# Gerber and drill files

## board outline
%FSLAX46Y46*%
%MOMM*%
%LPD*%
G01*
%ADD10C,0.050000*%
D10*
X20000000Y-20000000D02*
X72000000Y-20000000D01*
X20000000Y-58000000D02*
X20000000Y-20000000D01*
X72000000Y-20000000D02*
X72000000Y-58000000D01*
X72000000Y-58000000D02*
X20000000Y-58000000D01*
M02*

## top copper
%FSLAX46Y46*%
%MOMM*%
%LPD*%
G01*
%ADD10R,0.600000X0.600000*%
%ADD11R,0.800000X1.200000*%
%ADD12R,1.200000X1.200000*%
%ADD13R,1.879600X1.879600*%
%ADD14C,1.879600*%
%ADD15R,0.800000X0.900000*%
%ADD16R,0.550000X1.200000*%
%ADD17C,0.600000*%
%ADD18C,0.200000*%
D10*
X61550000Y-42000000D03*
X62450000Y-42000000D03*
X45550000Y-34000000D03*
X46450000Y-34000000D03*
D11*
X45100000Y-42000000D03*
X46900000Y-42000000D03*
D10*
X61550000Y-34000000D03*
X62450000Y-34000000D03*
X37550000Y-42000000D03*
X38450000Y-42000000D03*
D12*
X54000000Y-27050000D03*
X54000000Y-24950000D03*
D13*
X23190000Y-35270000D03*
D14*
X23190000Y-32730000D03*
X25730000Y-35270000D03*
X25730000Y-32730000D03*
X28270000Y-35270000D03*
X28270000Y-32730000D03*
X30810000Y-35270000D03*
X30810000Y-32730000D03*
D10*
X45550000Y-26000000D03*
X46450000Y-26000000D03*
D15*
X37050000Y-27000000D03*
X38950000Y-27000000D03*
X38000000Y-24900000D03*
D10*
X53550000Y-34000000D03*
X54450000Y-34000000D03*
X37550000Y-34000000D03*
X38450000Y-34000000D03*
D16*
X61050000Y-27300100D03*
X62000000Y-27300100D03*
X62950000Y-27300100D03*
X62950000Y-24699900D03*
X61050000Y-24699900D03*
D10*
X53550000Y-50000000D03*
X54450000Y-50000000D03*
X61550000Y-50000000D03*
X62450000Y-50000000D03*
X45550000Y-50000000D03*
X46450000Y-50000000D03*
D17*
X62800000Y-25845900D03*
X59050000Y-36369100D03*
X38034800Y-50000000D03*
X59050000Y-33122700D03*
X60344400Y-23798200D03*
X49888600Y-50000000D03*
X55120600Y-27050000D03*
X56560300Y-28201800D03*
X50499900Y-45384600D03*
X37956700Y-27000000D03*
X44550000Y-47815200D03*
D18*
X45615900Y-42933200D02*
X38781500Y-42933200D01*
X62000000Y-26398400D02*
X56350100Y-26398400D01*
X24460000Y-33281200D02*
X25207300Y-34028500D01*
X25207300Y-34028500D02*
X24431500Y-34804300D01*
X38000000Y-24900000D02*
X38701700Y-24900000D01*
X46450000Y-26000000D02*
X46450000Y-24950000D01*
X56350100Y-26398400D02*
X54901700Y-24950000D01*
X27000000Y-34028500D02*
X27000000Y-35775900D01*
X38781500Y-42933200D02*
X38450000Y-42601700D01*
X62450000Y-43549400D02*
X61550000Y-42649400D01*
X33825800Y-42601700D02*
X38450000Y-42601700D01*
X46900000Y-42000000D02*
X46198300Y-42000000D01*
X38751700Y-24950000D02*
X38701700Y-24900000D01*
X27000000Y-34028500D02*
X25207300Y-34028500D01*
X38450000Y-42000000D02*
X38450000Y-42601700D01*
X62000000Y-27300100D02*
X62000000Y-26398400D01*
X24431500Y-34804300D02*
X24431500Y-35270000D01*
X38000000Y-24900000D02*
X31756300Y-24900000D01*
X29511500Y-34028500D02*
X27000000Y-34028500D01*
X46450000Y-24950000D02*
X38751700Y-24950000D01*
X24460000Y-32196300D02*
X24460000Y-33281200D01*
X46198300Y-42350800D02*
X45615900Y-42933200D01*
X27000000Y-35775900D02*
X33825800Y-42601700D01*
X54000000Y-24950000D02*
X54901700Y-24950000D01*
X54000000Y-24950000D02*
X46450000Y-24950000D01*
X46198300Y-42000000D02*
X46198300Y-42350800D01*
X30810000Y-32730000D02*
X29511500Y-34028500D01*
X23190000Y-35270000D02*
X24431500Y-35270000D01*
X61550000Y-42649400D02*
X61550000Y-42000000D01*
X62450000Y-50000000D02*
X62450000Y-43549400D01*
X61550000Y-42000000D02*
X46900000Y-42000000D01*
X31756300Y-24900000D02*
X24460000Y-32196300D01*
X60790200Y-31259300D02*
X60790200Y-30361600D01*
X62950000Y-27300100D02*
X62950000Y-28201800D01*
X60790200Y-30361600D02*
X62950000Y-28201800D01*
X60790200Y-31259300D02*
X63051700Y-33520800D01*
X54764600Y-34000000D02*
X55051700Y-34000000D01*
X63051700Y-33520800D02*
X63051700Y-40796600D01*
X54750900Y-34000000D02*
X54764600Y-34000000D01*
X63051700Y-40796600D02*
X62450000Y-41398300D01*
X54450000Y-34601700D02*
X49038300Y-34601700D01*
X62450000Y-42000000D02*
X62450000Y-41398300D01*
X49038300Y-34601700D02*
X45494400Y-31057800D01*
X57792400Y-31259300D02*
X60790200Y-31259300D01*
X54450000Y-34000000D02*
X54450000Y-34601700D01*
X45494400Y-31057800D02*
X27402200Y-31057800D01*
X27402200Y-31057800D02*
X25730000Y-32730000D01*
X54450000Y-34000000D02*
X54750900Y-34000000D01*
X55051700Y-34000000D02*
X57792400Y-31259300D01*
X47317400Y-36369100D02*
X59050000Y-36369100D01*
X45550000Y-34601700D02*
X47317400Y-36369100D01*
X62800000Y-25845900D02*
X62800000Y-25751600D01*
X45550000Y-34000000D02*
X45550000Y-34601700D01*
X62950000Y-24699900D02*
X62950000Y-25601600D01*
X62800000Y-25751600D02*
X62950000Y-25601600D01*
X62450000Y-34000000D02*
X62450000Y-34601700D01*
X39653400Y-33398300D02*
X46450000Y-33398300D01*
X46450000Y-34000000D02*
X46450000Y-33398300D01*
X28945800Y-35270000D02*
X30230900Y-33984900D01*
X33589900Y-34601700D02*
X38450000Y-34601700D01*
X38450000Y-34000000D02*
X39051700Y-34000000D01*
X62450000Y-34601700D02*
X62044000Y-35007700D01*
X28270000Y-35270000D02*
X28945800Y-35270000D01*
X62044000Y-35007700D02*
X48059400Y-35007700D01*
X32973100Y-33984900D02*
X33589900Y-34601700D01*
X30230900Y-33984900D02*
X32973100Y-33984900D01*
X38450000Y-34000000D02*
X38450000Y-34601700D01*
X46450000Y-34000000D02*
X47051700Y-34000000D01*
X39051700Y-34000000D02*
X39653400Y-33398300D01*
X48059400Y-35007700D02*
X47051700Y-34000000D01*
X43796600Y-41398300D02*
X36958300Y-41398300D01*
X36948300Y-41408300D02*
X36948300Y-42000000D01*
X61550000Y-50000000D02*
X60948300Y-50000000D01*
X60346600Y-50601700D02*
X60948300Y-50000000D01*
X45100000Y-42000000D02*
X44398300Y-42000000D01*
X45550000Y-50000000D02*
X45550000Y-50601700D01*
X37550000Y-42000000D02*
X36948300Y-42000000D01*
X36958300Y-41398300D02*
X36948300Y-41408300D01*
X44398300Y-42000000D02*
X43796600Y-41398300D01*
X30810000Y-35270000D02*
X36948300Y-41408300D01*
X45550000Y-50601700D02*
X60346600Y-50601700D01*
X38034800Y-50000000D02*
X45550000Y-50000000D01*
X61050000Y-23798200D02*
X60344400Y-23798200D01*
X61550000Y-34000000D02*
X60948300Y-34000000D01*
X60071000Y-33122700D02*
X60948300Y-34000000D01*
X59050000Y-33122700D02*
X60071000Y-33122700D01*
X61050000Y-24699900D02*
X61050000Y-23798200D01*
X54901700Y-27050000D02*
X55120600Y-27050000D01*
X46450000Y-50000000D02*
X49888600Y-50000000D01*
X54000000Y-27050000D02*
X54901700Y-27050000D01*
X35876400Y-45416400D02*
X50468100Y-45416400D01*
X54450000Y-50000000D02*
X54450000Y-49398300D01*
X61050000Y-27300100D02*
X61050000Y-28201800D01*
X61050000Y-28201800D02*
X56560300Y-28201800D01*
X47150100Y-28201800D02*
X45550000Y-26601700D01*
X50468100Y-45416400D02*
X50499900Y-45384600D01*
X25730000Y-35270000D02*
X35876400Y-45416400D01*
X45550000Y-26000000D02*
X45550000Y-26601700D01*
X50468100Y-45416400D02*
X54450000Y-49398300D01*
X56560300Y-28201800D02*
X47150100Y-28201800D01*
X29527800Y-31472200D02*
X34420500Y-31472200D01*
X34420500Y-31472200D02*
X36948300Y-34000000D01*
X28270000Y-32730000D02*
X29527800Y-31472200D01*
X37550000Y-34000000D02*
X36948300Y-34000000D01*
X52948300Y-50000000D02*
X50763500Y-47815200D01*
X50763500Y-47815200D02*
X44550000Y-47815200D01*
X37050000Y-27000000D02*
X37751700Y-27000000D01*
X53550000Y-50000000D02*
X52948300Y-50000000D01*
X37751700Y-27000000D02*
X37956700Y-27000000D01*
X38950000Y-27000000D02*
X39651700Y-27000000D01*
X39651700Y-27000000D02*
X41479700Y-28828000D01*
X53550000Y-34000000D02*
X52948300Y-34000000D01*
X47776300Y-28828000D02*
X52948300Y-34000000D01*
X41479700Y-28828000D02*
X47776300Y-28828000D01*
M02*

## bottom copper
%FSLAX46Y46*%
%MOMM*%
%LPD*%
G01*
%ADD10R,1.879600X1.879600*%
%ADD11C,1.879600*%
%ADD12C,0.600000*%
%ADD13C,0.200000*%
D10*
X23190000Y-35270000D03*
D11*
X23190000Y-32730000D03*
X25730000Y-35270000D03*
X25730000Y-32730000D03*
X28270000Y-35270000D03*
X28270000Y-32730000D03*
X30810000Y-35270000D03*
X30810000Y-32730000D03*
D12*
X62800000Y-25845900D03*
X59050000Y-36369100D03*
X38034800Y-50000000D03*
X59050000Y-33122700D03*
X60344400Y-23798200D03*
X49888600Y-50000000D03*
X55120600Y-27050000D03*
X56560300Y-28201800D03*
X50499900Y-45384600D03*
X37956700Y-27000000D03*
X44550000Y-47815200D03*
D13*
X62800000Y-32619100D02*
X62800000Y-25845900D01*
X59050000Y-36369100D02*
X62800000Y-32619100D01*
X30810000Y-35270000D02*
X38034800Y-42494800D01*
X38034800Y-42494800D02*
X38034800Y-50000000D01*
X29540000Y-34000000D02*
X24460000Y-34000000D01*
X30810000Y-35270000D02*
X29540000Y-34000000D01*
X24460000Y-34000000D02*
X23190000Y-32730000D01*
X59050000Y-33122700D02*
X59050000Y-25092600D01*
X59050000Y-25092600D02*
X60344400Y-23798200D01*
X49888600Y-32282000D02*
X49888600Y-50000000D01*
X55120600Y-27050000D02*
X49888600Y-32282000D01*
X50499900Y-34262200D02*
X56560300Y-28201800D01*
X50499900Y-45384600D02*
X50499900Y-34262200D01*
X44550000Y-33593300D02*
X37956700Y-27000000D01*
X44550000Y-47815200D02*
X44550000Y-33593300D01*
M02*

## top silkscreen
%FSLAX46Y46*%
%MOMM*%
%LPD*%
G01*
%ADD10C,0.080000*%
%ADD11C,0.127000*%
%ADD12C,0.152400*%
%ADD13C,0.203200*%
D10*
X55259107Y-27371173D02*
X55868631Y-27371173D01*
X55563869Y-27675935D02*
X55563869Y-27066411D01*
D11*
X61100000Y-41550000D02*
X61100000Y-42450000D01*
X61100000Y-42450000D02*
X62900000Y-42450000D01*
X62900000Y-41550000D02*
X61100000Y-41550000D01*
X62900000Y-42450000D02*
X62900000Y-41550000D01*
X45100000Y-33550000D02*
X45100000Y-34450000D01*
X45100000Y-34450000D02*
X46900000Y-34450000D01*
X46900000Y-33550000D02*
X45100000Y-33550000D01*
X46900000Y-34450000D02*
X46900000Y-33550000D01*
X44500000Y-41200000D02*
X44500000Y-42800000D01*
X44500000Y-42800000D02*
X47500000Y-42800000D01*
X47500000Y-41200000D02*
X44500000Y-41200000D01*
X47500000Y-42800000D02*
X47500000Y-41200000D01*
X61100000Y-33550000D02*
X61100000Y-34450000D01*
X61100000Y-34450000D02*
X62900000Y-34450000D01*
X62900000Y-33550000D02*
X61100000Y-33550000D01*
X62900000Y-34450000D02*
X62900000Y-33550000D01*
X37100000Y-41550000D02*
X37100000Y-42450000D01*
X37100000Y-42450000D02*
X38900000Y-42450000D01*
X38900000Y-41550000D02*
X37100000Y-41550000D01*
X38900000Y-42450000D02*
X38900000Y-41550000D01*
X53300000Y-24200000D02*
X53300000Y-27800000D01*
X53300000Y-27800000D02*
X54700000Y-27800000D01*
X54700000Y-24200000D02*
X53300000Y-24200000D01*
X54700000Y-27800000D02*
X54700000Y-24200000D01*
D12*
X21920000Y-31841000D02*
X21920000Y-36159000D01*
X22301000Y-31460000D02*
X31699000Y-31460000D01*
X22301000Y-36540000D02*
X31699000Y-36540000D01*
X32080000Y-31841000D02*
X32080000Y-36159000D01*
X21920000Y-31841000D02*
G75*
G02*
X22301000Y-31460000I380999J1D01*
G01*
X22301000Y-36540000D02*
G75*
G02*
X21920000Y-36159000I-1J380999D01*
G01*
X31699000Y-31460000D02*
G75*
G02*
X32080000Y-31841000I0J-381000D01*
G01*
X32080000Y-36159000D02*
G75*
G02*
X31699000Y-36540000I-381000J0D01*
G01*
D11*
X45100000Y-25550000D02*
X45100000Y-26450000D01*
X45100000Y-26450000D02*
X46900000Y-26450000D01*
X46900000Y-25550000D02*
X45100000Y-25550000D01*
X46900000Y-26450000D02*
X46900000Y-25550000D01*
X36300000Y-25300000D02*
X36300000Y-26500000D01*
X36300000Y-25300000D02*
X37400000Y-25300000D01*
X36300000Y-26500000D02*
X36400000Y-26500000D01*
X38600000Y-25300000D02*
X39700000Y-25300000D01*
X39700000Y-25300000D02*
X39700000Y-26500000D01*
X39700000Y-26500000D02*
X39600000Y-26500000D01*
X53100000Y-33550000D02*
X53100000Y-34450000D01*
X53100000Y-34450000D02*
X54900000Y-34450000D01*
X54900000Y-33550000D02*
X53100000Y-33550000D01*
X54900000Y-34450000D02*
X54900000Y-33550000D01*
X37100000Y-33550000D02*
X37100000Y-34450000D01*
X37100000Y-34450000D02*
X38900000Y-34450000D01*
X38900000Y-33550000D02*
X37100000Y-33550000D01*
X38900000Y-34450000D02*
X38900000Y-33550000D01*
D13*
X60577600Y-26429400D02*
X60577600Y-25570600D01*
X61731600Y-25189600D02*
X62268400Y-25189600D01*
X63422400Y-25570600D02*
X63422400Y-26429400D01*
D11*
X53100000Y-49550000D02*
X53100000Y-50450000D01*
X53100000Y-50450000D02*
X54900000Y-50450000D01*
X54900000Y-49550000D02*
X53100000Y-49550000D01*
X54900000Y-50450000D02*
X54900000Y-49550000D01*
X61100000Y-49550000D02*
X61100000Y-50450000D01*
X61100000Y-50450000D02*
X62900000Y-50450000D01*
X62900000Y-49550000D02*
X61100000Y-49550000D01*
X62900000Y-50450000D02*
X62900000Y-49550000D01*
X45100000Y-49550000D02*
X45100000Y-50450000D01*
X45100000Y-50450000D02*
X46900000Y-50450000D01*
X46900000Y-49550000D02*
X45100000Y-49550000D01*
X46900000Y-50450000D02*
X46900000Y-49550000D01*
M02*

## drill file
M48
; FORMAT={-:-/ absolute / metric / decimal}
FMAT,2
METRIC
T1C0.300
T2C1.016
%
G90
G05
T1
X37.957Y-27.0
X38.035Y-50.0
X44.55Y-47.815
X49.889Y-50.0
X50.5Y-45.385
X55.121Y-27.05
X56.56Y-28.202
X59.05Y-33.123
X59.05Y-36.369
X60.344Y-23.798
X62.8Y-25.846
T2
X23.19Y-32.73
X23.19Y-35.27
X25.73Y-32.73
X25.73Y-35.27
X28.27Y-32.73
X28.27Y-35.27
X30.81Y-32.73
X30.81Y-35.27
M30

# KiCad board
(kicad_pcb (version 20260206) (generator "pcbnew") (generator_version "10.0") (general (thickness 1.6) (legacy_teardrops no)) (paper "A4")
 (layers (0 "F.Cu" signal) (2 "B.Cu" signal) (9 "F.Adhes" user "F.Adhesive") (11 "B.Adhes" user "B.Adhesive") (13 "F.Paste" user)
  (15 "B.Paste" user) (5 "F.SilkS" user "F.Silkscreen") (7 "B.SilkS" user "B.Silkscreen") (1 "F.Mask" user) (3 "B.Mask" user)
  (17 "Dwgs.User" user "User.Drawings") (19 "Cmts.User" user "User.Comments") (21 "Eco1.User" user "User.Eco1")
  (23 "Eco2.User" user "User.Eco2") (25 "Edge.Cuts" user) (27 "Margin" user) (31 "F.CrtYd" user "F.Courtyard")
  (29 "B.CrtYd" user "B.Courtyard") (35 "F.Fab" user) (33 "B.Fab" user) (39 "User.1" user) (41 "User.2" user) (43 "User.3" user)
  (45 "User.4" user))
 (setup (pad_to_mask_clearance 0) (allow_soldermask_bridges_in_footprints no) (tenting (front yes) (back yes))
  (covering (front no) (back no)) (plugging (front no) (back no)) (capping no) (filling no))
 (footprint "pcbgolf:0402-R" (layer "F.Cu") (at 62 42)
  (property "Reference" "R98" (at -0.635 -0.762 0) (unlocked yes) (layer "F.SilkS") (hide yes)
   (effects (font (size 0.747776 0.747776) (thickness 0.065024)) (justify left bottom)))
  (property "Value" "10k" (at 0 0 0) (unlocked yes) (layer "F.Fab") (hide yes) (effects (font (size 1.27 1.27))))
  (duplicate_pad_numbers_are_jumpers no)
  (fp_line (start -0.9 -0.45) (end -0.9 0.45) (stroke (width 0.127) (type solid)) (layer "F.SilkS"))
  (fp_line (start -0.9 0.45) (end 0.9 0.45) (stroke (width 0.127) (type solid)) (layer "F.SilkS"))
  (fp_line (start 0.9 -0.45) (end -0.9 -0.45) (stroke (width 0.127) (type solid)) (layer "F.SilkS"))
  (fp_line (start 0.9 0.45) (end 0.9 -0.45) (stroke (width 0.127) (type solid)) (layer "F.SilkS"))
  (pad "1" smd rect (at -0.45 0) (size 0.6 0.6) (layers "F.Cu" "F.Mask" "F.Paste") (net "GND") (solder_mask_margin 0.0508)
   (solder_paste_margin 0) (thermal_bridge_angle 0))
  (pad "2" smd rect (at 0.45 0) (size 0.6 0.6) (layers "F.Cu" "F.Mask" "F.Paste") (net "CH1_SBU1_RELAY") (solder_mask_margin 0.0508)
   (solder_paste_margin 0) (thermal_bridge_angle 0)))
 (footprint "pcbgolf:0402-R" (layer "F.Cu") (at 46 34)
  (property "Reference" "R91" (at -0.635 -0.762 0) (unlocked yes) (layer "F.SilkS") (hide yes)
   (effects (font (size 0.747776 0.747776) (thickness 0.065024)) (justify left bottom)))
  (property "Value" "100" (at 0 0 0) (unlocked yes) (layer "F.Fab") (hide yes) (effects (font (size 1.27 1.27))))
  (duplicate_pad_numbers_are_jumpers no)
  (fp_line (start -0.9 -0.45) (end -0.9 0.45) (stroke (width 0.127) (type solid)) (layer "F.SilkS"))
  (fp_line (start -0.9 0.45) (end 0.9 0.45) (stroke (width 0.127) (type solid)) (layer "F.SilkS"))
  (fp_line (start 0.9 -0.45) (end -0.9 -0.45) (stroke (width 0.127) (type solid)) (layer "F.SilkS"))
  (fp_line (start 0.9 0.45) (end 0.9 -0.45) (stroke (width 0.127) (type solid)) (layer "F.SilkS"))
  (pad "1" smd rect (at -0.45 0) (size 0.6 0.6) (layers "F.Cu" "F.Mask" "F.Paste") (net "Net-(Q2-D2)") (solder_mask_margin 0.0508)
   (solder_paste_margin 0) (thermal_bridge_angle 0))
  (pad "2" smd rect (at 0.45 0) (size 0.6 0.6) (layers "F.Cu" "F.Mask" "F.Paste") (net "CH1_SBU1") (solder_mask_margin 0.0508)
   (solder_paste_margin 0) (thermal_bridge_angle 0)))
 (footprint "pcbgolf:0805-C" (layer "F.Cu") (at 46 42)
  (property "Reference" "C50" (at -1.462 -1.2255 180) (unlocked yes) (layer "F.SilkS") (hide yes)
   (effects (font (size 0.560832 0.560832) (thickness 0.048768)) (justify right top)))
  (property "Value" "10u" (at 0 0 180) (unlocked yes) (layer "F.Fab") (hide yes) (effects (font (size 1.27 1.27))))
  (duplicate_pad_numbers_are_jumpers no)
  (fp_line (start -1.5 -0.8) (end -1.5 0.8) (stroke (width 0.127) (type solid)) (layer "F.SilkS"))
  (fp_line (start -1.5 0.8) (end 1.5 0.8) (stroke (width 0.127) (type solid)) (layer "F.SilkS"))
  (fp_line (start 1.5 -0.8) (end -1.5 -0.8) (stroke (width 0.127) (type solid)) (layer "F.SilkS"))
  (fp_line (start 1.5 0.8) (end 1.5 -0.8) (stroke (width 0.127) (type solid)) (layer "F.SilkS"))
  (pad "1" smd rect (at -0.9 0) (size 0.8 1.2) (layers "F.Cu" "F.Mask" "F.Paste") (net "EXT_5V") (solder_mask_margin 0.0508)
   (solder_paste_margin 0) (thermal_bridge_angle 0))
  (pad "2" smd rect (at 0.9 0) (size 0.8 1.2) (layers "F.Cu" "F.Mask" "F.Paste") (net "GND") (solder_mask_margin 0.0508)
   (solder_paste_margin 0) (thermal_bridge_angle 0)))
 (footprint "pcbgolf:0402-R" (layer "F.Cu") (at 62 34)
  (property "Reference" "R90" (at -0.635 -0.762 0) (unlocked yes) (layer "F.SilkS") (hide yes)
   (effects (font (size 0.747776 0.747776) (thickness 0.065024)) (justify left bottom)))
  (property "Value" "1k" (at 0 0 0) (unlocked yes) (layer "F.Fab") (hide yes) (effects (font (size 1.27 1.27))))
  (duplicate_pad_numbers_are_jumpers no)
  (fp_line (start -0.9 -0.45) (end -0.9 0.45) (stroke (width 0.127) (type solid)) (layer "F.SilkS"))
  (fp_line (start -0.9 0.45) (end 0.9 0.45) (stroke (width 0.127) (type solid)) (layer "F.SilkS"))
  (fp_line (start 0.9 -0.45) (end -0.9 -0.45) (stroke (width 0.127) (type solid)) (layer "F.SilkS"))
  (fp_line (start 0.9 0.45) (end 0.9 -0.45) (stroke (width 0.127) (type solid)) (layer "F.SilkS"))
  (pad "1" smd rect (at -0.45 0) (size 0.6 0.6) (layers "F.Cu" "F.Mask" "F.Paste") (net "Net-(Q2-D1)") (solder_mask_margin 0.0508)
   (solder_paste_margin 0) (thermal_bridge_angle 0))
  (pad "2" smd rect (at 0.45 0) (size 0.6 0.6) (layers "F.Cu" "F.Mask" "F.Paste") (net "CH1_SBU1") (solder_mask_margin 0.0508)
   (solder_paste_margin 0) (thermal_bridge_angle 0)))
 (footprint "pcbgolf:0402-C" (layer "F.Cu") (at 38 42)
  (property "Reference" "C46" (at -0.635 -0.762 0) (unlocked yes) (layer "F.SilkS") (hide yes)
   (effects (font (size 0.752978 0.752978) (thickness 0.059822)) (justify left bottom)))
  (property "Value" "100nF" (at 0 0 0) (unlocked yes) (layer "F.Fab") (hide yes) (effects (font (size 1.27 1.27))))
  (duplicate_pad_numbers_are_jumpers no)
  (fp_line (start -0.9 -0.45) (end -0.9 0.45) (stroke (width 0.127) (type solid)) (layer "F.SilkS"))
  (fp_line (start -0.9 0.45) (end 0.9 0.45) (stroke (width 0.127) (type solid)) (layer "F.SilkS"))
  (fp_line (start 0.9 -0.45) (end -0.9 -0.45) (stroke (width 0.127) (type solid)) (layer "F.SilkS"))
  (fp_line (start 0.9 0.45) (end 0.9 -0.45) (stroke (width 0.127) (type solid)) (layer "F.SilkS"))
  (pad "1" smd rect (at -0.45 0) (size 0.6 0.6) (layers "F.Cu" "F.Mask" "F.Paste") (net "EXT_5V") (solder_mask_margin 0.0508)
   (solder_paste_margin 0) (thermal_bridge_angle 0))
  (pad "2" smd rect (at 0.45 0) (size 0.6 0.6) (layers "F.Cu" "F.Mask" "F.Paste") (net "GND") (solder_mask_margin 0.0508)
   (solder_paste_margin 0) (thermal_bridge_angle 0)))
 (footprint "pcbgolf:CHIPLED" (layer "F.Cu") (at 54 26)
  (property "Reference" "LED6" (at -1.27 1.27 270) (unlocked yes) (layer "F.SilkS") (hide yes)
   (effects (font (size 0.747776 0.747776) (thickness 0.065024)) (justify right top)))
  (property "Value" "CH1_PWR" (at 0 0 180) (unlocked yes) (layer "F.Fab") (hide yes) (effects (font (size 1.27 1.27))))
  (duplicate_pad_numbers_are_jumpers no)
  (fp_line (start -0.7 -1.8) (end -0.7 1.8) (stroke (width 0.127) (type solid)) (layer "F.SilkS"))
  (fp_line (start -0.7 1.8) (end 0.7 1.8) (stroke (width 0.127) (type solid)) (layer "F.SilkS"))
  (fp_line (start 0.7 -1.8) (end -0.7 -1.8) (stroke (width 0.127) (type solid)) (layer "F.SilkS"))
  (fp_line (start 0.7 1.8) (end 0.7 -1.8) (stroke (width 0.127) (type solid)) (layer "F.SilkS"))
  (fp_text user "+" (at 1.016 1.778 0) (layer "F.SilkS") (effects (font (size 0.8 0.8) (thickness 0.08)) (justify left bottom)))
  (pad "A" smd rect (at 0 1.05) (size 1.2 1.2) (layers "F.Cu" "F.Mask" "F.Paste") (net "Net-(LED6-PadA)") (solder_mask_margin 0.0508)
   (solder_paste_margin 0) (thermal_bridge_angle 0))
  (pad "C" smd rect (at 0 -1.05) (size 1.2 1.2) (layers "F.Cu" "F.Mask" "F.Paste") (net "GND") (solder_mask_margin 0.0508)
   (solder_paste_margin 0) (thermal_bridge_angle 0)))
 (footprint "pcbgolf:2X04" (layer "F.Cu") (at 27 34)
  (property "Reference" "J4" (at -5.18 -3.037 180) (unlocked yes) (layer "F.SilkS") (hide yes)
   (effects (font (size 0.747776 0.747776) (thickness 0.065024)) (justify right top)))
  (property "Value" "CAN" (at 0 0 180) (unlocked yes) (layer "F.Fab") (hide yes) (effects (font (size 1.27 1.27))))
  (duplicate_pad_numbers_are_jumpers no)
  (fp_line (start -5.08 -2.159) (end -5.08 2.159) (stroke (width 0.1524) (type solid)) (layer "F.SilkS"))
  (fp_line (start -4.699 -2.54) (end 4.699 -2.54) (stroke (width 0.1524) (type solid)) (layer "F.SilkS"))
  (fp_line (start -4.699 2.54) (end 4.699 2.54) (stroke (width 0.1524) (type solid)) (layer "F.SilkS"))
  (fp_line (start 5.08 -2.159) (end 5.08 2.159) (stroke (width 0.1524) (type solid)) (layer "F.SilkS"))
  (fp_arc (start -5.08 -2.159) (mid -4.968408 -2.428408) (end -4.699 -2.54) (stroke (width 0.1524) (type solid)) (layer "F.SilkS"))
  (fp_arc (start -4.699 2.54) (mid -4.968408 2.428408) (end -5.08 2.159) (stroke (width 0.1524) (type solid)) (layer "F.SilkS"))
  (fp_arc (start 4.699 -2.54) (mid 4.968408 -2.428408) (end 5.08 -2.159) (stroke (width 0.1524) (type solid)) (layer "F.SilkS"))
  (fp_arc (start 5.08 2.159) (mid 4.968408 2.428408) (end 4.699 2.54) (stroke (width 0.1524) (type solid)) (layer "F.SilkS"))
  (pad "1" thru_hole rect (at -3.81 1.27 90) (size 1.8796 1.8796) (drill 1.016) (layers "*.Cu" "*.Mask") (remove_unused_layers no)
   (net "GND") (solder_mask_margin 0.0508) (thermal_bridge_angle 0))
  (pad "2" thru_hole circle (at -3.81 -1.27 90) (size 1.8796 1.8796) (drill 1.016) (layers "*.Cu" "*.Mask") (remove_unused_layers no)
   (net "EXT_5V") (solder_mask_margin 0.0508) (thermal_bridge_angle 0))
  (pad "3" thru_hole circle (at -1.27 1.27 90) (size 1.8796 1.8796) (drill 1.016) (layers "*.Cu" "*.Mask") (remove_unused_layers no)
   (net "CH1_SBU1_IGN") (solder_mask_margin 0.0508) (thermal_bridge_angle 0))
  (pad "4" thru_hole circle (at -1.27 -1.27 90) (size 1.8796 1.8796) (drill 1.016) (layers "*.Cu" "*.Mask") (remove_unused_layers no)
   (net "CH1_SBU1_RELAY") (solder_mask_margin 0.0508) (thermal_bridge_angle 0))
  (pad "5" thru_hole circle (at 1.27 1.27 90) (size 1.8796 1.8796) (drill 1.016) (layers "*.Cu" "*.Mask") (remove_unused_layers no)
   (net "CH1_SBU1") (solder_mask_margin 0.0508) (thermal_bridge_angle 0))
  (pad "6" thru_hole circle (at 1.27 -1.27 90) (size 1.8796 1.8796) (drill 1.016) (layers "*.Cu" "*.Mask") (remove_unused_layers no)
   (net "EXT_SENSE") (solder_mask_margin 0.0508) (thermal_bridge_angle 0))
  (pad "7" thru_hole circle (at 3.81 1.27 90) (size 1.8796 1.8796) (drill 1.016) (layers "*.Cu" "*.Mask") (remove_unused_layers no)
   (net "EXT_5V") (solder_mask_margin 0.0508) (thermal_bridge_angle 0))
  (pad "8" thru_hole circle (at 3.81 -1.27 90) (size 1.8796 1.8796) (drill 1.016) (layers "*.Cu" "*.Mask") (remove_unused_layers no)
   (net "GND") (solder_mask_margin 0.0508) (thermal_bridge_angle 0)))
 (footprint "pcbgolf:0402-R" (layer "F.Cu") (at 46 26)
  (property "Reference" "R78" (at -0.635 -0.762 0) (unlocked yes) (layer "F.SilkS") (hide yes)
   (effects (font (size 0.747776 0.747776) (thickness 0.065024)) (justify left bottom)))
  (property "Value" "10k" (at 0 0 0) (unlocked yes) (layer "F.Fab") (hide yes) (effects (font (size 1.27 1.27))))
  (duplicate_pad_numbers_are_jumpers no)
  (fp_line (start -0.9 -0.45) (end -0.9 0.45) (stroke (width 0.127) (type solid)) (layer "F.SilkS"))
  (fp_line (start -0.9 0.45) (end 0.9 0.45) (stroke (width 0.127) (type solid)) (layer "F.SilkS"))
  (fp_line (start 0.9 -0.45) (end -0.9 -0.45) (stroke (width 0.127) (type solid)) (layer "F.SilkS"))
  (fp_line (start 0.9 0.45) (end 0.9 -0.45) (stroke (width 0.127) (type solid)) (layer "F.SilkS"))
  (pad "1" smd rect (at -0.45 0) (size 0.6 0.6) (layers "F.Cu" "F.Mask" "F.Paste") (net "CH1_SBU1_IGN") (solder_mask_margin 0.0508)
   (solder_paste_margin 0) (thermal_bridge_angle 0))
  (pad "2" smd rect (at 0.45 0) (size 0.6 0.6) (layers "F.Cu" "F.Mask" "F.Paste") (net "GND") (solder_mask_margin 0.0508)
   (solder_paste_margin 0) (thermal_bridge_angle 0)))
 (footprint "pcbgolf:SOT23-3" (layer "F.Cu") (at 38 26)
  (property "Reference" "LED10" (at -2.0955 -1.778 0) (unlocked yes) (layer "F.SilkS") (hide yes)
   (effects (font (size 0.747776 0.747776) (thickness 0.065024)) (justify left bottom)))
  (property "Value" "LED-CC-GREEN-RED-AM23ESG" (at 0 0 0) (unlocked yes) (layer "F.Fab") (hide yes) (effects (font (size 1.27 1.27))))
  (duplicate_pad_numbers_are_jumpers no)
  (fp_line (start -1.7 -0.7) (end -1.7 0.5) (stroke (width 0.127) (type solid)) (layer "F.SilkS"))
  (fp_line (start -1.7 -0.7) (end -0.6 -0.7) (stroke (width 0.127) (type solid)) (layer "F.SilkS"))
  (fp_line (start -1.7 0.5) (end -1.6 0.5) (stroke (width 0.127) (type solid)) (layer "F.SilkS"))
  (fp_line (start 0.6 -0.7) (end 1.7 -0.7) (stroke (width 0.127) (type solid)) (layer "F.SilkS"))
  (fp_line (start 1.7 -0.7) (end 1.7 0.5) (stroke (width 0.127) (type solid)) (layer "F.SilkS"))
  (fp_line (start 1.7 0.5) (end 1.6 0.5) (stroke (width 0.127) (type solid)) (layer "F.SilkS"))
  (pad "1" smd rect (at -0.95 1) (size 0.8 0.9) (layers "F.Cu" "F.Mask" "F.Paste") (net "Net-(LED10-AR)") (solder_mask_margin 0.0508)
   (solder_paste_margin 0) (thermal_bridge_angle 0))
  (pad "2" smd rect (at 0.95 1) (size 0.8 0.9) (layers "F.Cu" "F.Mask" "F.Paste") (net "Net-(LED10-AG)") (solder_mask_margin 0.0508)
   (solder_paste_margin 0) (thermal_bridge_angle 0))
  (pad "3" smd rect (at 0 -1.1) (size 0.8 0.9) (layers "F.Cu" "F.Mask" "F.Paste") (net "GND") (solder_mask_margin 0.0508)
   (solder_paste_margin 0) (thermal_bridge_angle 0)))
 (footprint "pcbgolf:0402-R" (layer "F.Cu") (at 54 34)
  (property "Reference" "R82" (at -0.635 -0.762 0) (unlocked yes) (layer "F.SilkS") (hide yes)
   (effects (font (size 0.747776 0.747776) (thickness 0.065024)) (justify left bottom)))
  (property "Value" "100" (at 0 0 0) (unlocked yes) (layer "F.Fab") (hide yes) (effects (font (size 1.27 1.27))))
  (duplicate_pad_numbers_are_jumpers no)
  (fp_line (start -0.9 -0.45) (end -0.9 0.45) (stroke (width 0.127) (type solid)) (layer "F.SilkS"))
  (fp_line (start -0.9 0.45) (end 0.9 0.45) (stroke (width 0.127) (type solid)) (layer "F.SilkS"))
  (fp_line (start 0.9 -0.45) (end -0.9 -0.45) (stroke (width 0.127) (type solid)) (layer "F.SilkS"))
  (fp_line (start 0.9 0.45) (end 0.9 -0.45) (stroke (width 0.127) (type solid)) (layer "F.SilkS"))
  (pad "1" smd rect (at -0.45 0) (size 0.6 0.6) (layers "F.Cu" "F.Mask" "F.Paste") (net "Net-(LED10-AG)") (solder_mask_margin 0.0508)
   (solder_paste_margin 0) (thermal_bridge_angle 0))
  (pad "2" smd rect (at 0.45 0) (size 0.6 0.6) (layers "F.Cu" "F.Mask" "F.Paste") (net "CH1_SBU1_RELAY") (solder_mask_margin 0.0508)
   (solder_paste_margin 0) (thermal_bridge_angle 0)))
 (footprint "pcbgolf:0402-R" (layer "F.Cu") (at 38 34)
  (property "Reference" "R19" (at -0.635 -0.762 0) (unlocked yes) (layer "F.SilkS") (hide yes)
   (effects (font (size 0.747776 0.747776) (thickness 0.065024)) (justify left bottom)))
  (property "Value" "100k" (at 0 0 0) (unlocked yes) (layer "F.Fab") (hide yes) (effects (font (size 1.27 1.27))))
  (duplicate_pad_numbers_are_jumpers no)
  (fp_line (start -0.9 -0.45) (end -0.9 0.45) (stroke (width 0.127) (type solid)) (layer "F.SilkS"))
  (fp_line (start -0.9 0.45) (end 0.9 0.45) (stroke (width 0.127) (type solid)) (layer "F.SilkS"))
  (fp_line (start 0.9 -0.45) (end -0.9 -0.45) (stroke (width 0.127) (type solid)) (layer "F.SilkS"))
  (fp_line (start 0.9 0.45) (end 0.9 -0.45) (stroke (width 0.127) (type solid)) (layer "F.SilkS"))
  (pad "1" smd rect (at -0.45 0) (size 0.6 0.6) (layers "F.Cu" "F.Mask" "F.Paste") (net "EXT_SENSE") (solder_mask_margin 0.0508)
   (solder_paste_margin 0) (thermal_bridge_angle 0))
  (pad "2" smd rect (at 0.45 0) (size 0.6 0.6) (layers "F.Cu" "F.Mask" "F.Paste") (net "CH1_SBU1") (solder_mask_margin 0.0508)
   (solder_paste_margin 0) (thermal_bridge_angle 0)))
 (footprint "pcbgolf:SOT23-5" (layer "F.Cu") (at 62 26)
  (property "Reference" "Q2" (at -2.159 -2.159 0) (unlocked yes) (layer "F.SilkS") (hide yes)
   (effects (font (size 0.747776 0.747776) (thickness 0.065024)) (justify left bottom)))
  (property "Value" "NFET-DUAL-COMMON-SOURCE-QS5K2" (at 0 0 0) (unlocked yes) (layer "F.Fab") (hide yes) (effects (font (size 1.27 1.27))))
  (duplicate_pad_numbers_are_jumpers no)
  (fp_line (start -1.4224 0.4294) (end -1.4224 -0.4294) (stroke (width 0.2032) (type solid)) (layer "F.SilkS"))
  (fp_line (start -0.2684 -0.8104) (end 0.2684 -0.8104) (stroke (width 0.2032) (type solid)) (layer "F.SilkS"))
  (fp_line (start 1.4224 -0.4294) (end 1.4224 0.4294) (stroke (width 0.2032) (type solid)) (layer "F.SilkS"))
  (pad "1" smd rect (at -0.95 1.3001) (size 0.55 1.2) (layers "F.Cu" "F.Mask" "F.Paste") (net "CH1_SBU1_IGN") (solder_mask_margin 0.0508)
   (solder_paste_margin 0) (thermal_bridge_angle 0))
  (pad "2" smd rect (at 0 1.3001) (size 0.55 1.2) (layers "F.Cu" "F.Mask" "F.Paste") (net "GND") (solder_mask_margin 0.0508)
   (solder_paste_margin 0) (thermal_bridge_angle 0))
  (pad "3" smd rect (at 0.95 1.3001) (size 0.55 1.2) (layers "F.Cu" "F.Mask" "F.Paste") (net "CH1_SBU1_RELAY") (solder_mask_margin 0.0508)
   (solder_paste_margin 0) (thermal_bridge_angle 0))
  (pad "4" smd rect (at 0.95 -1.3001) (size 0.55 1.2) (layers "F.Cu" "F.Mask" "F.Paste") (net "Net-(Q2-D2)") (solder_mask_margin 0.0508)
   (solder_paste_margin 0) (thermal_bridge_angle 0))
  (pad "5" smd rect (at -0.95 -1.3001) (size 0.55 1.2) (layers "F.Cu" "F.Mask" "F.Paste") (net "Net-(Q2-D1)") (solder_mask_margin 0.0508)
   (solder_paste_margin 0) (thermal_bridge_angle 0)))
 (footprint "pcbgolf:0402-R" (layer "F.Cu") (at 54 50)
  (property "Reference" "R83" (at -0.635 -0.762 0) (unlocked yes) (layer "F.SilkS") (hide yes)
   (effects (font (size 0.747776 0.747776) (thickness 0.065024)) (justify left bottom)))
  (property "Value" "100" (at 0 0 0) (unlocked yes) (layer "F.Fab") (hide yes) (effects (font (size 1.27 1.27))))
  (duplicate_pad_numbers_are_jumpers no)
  (fp_line (start -0.9 -0.45) (end -0.9 0.45) (stroke (width 0.127) (type solid)) (layer "F.SilkS"))
  (fp_line (start -0.9 0.45) (end 0.9 0.45) (stroke (width 0.127) (type solid)) (layer "F.SilkS"))
  (fp_line (start 0.9 -0.45) (end -0.9 -0.45) (stroke (width 0.127) (type solid)) (layer "F.SilkS"))
  (fp_line (start 0.9 0.45) (end 0.9 -0.45) (stroke (width 0.127) (type solid)) (layer "F.SilkS"))
  (pad "1" smd rect (at -0.45 0) (size 0.6 0.6) (layers "F.Cu" "F.Mask" "F.Paste") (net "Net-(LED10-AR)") (solder_mask_margin 0.0508)
   (solder_paste_margin 0) (thermal_bridge_angle 0))
  (pad "2" smd rect (at 0.45 0) (size 0.6 0.6) (layers "F.Cu" "F.Mask" "F.Paste") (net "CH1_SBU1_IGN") (solder_mask_margin 0.0508)
   (solder_paste_margin 0) (thermal_bridge_angle 0)))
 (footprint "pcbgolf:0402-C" (layer "F.Cu") (at 62 50)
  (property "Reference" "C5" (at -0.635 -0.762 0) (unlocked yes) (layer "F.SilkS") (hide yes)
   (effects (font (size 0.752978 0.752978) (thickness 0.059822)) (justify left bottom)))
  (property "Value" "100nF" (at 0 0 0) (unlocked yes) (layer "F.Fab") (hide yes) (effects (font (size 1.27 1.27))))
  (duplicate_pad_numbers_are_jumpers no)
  (fp_line (start -0.9 -0.45) (end -0.9 0.45) (stroke (width 0.127) (type solid)) (layer "F.SilkS"))
  (fp_line (start -0.9 0.45) (end 0.9 0.45) (stroke (width 0.127) (type solid)) (layer "F.SilkS"))
  (fp_line (start 0.9 -0.45) (end -0.9 -0.45) (stroke (width 0.127) (type solid)) (layer "F.SilkS"))
  (fp_line (start 0.9 0.45) (end 0.9 -0.45) (stroke (width 0.127) (type solid)) (layer "F.SilkS"))
  (pad "1" smd rect (at -0.45 0) (size 0.6 0.6) (layers "F.Cu" "F.Mask" "F.Paste") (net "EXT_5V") (solder_mask_margin 0.0508)
   (solder_paste_margin 0) (thermal_bridge_angle 0))
  (pad "2" smd rect (at 0.45 0) (size 0.6 0.6) (layers "F.Cu" "F.Mask" "F.Paste") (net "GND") (solder_mask_margin 0.0508)
   (solder_paste_margin 0) (thermal_bridge_angle 0)))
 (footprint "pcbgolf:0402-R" (layer "F.Cu") (at 46 50)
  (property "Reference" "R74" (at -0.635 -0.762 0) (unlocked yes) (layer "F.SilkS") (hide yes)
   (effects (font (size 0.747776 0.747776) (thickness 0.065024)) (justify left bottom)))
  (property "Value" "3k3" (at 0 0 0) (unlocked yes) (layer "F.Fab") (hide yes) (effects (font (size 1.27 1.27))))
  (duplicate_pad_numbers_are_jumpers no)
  (fp_line (start -0.9 -0.45) (end -0.9 0.45) (stroke (width 0.127) (type solid)) (layer "F.SilkS"))
  (fp_line (start -0.9 0.45) (end 0.9 0.45) (stroke (width 0.127) (type solid)) (layer "F.SilkS"))
  (fp_line (start 0.9 -0.45) (end -0.9 -0.45) (stroke (width 0.127) (type solid)) (layer "F.SilkS"))
  (fp_line (start 0.9 0.45) (end 0.9 -0.45) (stroke (width 0.127) (type solid)) (layer "F.SilkS"))
  (pad "1" smd rect (at -0.45 0) (size 0.6 0.6) (layers "F.Cu" "F.Mask" "F.Paste") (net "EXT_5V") (solder_mask_margin 0.0508)
   (solder_paste_margin 0) (thermal_bridge_angle 0))
  (pad "2" smd rect (at 0.45 0) (size 0.6 0.6) (layers "F.Cu" "F.Mask" "F.Paste") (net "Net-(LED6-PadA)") (solder_mask_margin 0.0508)
   (solder_paste_margin 0) (thermal_bridge_angle 0)))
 (gr_line (start 20 20) (end 72 20) (stroke (width 0.05) (type default)) (layer "Edge.Cuts"))
 (gr_line (start 20 58) (end 20 20) (stroke (width 0.05) (type default)) (layer "Edge.Cuts"))
 (gr_line (start 72 20) (end 72 58) (stroke (width 0.05) (type default)) (layer "Edge.Cuts"))
 (gr_line (start 72 58) (end 20 58) (stroke (width 0.05) (type default)) (layer "Edge.Cuts"))
 (segment (start 45.6159 42.9332) (end 38.7815 42.9332) (width 0.2) (layer "F.Cu") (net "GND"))
 (segment (start 62 26.3984) (end 56.3501 26.3984) (width 0.2) (layer "F.Cu") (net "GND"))
 (segment (start 24.46 33.2812) (end 25.2073 34.0285) (width 0.2) (layer "F.Cu") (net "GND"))
 (segment (start 25.2073 34.0285) (end 24.4315 34.8043) (width 0.2) (layer "F.Cu") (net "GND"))
 (segment (start 38 24.9) (end 38.7017 24.9) (width 0.2) (layer "F.Cu") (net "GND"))
 (segment (start 46.45 26) (end 46.45 24.95) (width 0.2) (layer "F.Cu") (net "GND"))
 (segment (start 56.3501 26.3984) (end 54.9017 24.95) (width 0.2) (layer "F.Cu") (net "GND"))
 (segment (start 27 34.0285) (end 27 35.7759) (width 0.2) (layer "F.Cu") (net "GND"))
 (segment (start 38.7815 42.9332) (end 38.45 42.6017) (width 0.2) (layer "F.Cu") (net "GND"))
 (segment (start 62.45 43.5494) (end 61.55 42.6494) (width 0.2) (layer "F.Cu") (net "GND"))
 (segment (start 33.8258 42.6017) (end 38.45 42.6017) (width 0.2) (layer "F.Cu") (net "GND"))
 (segment (start 46.9 42) (end 46.1983 42) (width 0.2) (layer "F.Cu") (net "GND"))
 (segment (start 38.7517 24.95) (end 38.7017 24.9) (width 0.2) (layer "F.Cu") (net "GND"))
 (segment (start 27 34.0285) (end 25.2073 34.0285) (width 0.2) (layer "F.Cu") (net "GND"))
 (segment (start 38.45 42) (end 38.45 42.6017) (width 0.2) (layer "F.Cu") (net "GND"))
 (segment (start 62 27.3001) (end 62 26.3984) (width 0.2) (layer "F.Cu") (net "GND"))
 (segment (start 24.4315 34.8043) (end 24.4315 35.27) (width 0.2) (layer "F.Cu") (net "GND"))
 (segment (start 38 24.9) (end 31.7563 24.9) (width 0.2) (layer "F.Cu") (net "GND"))
 (segment (start 29.5115 34.0285) (end 27 34.0285) (width 0.2) (layer "F.Cu") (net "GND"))
 (segment (start 46.45 24.95) (end 38.7517 24.95) (width 0.2) (layer "F.Cu") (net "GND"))
 (segment (start 24.46 32.1963) (end 24.46 33.2812) (width 0.2) (layer "F.Cu") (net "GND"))
 (segment (start 46.1983 42.3508) (end 45.6159 42.9332) (width 0.2) (layer "F.Cu") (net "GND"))
 (segment (start 27 35.7759) (end 33.8258 42.6017) (width 0.2) (layer "F.Cu") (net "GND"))
 (segment (start 54 24.95) (end 54.9017 24.95) (width 0.2) (layer "F.Cu") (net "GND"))
 (segment (start 54 24.95) (end 46.45 24.95) (width 0.2) (layer "F.Cu") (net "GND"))
 (segment (start 46.1983 42) (end 46.1983 42.3508) (width 0.2) (layer "F.Cu") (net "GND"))
 (segment (start 30.81 32.73) (end 29.5115 34.0285) (width 0.2) (layer "F.Cu") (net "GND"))
 (segment (start 23.19 35.27) (end 24.4315 35.27) (width 0.2) (layer "F.Cu") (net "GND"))
 (segment (start 61.55 42.6494) (end 61.55 42) (width 0.2) (layer "F.Cu") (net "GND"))
 (segment (start 62.45 50) (end 62.45 43.5494) (width 0.2) (layer "F.Cu") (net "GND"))
 (segment (start 61.55 42) (end 46.9 42) (width 0.2) (layer "F.Cu") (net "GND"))
 (segment (start 31.7563 24.9) (end 24.46 32.1963) (width 0.2) (layer "F.Cu") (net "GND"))
 (segment (start 60.7902 31.2593) (end 60.7902 30.3616) (width 0.2) (layer "F.Cu") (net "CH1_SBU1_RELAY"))
 (segment (start 62.95 27.3001) (end 62.95 28.2018) (width 0.2) (layer "F.Cu") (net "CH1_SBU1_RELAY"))
 (segment (start 60.7902 30.3616) (end 62.95 28.2018) (width 0.2) (layer "F.Cu") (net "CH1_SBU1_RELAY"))
 (segment (start 60.7902 31.2593) (end 63.0517 33.5208) (width 0.2) (layer "F.Cu") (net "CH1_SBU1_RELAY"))
 (segment (start 54.7646 34) (end 55.0517 34) (width 0.2) (layer "F.Cu") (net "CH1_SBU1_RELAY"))
 (segment (start 63.0517 33.5208) (end 63.0517 40.7966) (width 0.2) (layer "F.Cu") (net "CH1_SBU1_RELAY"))
 (segment (start 54.7509 34) (end 54.7646 34) (width 0.2) (layer "F.Cu") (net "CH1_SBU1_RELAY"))
 (segment (start 63.0517 40.7966) (end 62.45 41.3983) (width 0.2) (layer "F.Cu") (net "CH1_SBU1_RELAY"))
 (segment (start 54.45 34.6017) (end 49.0383 34.6017) (width 0.2) (layer "F.Cu") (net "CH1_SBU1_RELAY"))
 (segment (start 62.45 42) (end 62.45 41.3983) (width 0.2) (layer "F.Cu") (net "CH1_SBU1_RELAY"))
 (segment (start 49.0383 34.6017) (end 45.4944 31.0578) (width 0.2) (layer "F.Cu") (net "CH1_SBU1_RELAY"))
 (segment (start 57.7924 31.2593) (end 60.7902 31.2593) (width 0.2) (layer "F.Cu") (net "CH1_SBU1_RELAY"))
 (segment (start 54.45 34) (end 54.45 34.6017) (width 0.2) (layer "F.Cu") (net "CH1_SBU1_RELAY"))
 (segment (start 45.4944 31.0578) (end 27.4022 31.0578) (width 0.2) (layer "F.Cu") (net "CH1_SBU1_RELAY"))
 (segment (start 27.4022 31.0578) (end 25.73 32.73) (width 0.2) (layer "F.Cu") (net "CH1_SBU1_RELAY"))
 (segment (start 54.45 34) (end 54.7509 34) (width 0.2) (layer "F.Cu") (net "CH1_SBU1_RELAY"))
 (segment (start 55.0517 34) (end 57.7924 31.2593) (width 0.2) (layer "F.Cu") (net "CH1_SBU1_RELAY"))
 (segment (start 47.3174 36.3691) (end 59.05 36.3691) (width 0.2) (layer "F.Cu") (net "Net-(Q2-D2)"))
 (segment (start 45.55 34.6017) (end 47.3174 36.3691) (width 0.2) (layer "F.Cu") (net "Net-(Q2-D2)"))
 (segment (start 62.8 25.8459) (end 62.8 25.7516) (width 0.2) (layer "F.Cu") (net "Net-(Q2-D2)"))
 (segment (start 45.55 34) (end 45.55 34.6017) (width 0.2) (layer "F.Cu") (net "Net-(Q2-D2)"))
 (segment (start 62.95 24.6999) (end 62.95 25.6016) (width 0.2) (layer "F.Cu") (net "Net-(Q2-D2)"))
 (segment (start 62.8 25.7516) (end 62.95 25.6016) (width 0.2) (layer "F.Cu") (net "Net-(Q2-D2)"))
 (via (at 62.8 25.8459) (size 0.6) (drill 0.3) (layers "F.Cu" "B.Cu") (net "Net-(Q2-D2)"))
 (via (at 59.05 36.3691) (size 0.6) (drill 0.3) (layers "F.Cu" "B.Cu") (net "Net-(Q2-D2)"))
 (segment (start 62.8 32.6191) (end 62.8 25.8459) (width 0.2) (layer "B.Cu") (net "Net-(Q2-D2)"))
 (segment (start 59.05 36.3691) (end 62.8 32.6191) (width 0.2) (layer "B.Cu") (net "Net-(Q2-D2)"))
 (segment (start 62.45 34) (end 62.45 34.6017) (width 0.2) (layer "F.Cu") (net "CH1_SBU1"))
 (segment (start 39.6534 33.3983) (end 46.45 33.3983) (width 0.2) (layer "F.Cu") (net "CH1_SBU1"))
 (segment (start 46.45 34) (end 46.45 33.3983) (width 0.2) (layer "F.Cu") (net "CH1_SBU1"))
 (segment (start 28.9458 35.27) (end 30.2309 33.9849) (width 0.2) (layer "F.Cu") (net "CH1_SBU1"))
 (segment (start 33.5899 34.6017) (end 38.45 34.6017) (width 0.2) (layer "F.Cu") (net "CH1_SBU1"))
 (segment (start 38.45 34) (end 39.0517 34) (width 0.2) (layer "F.Cu") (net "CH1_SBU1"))
 (segment (start 62.45 34.6017) (end 62.044 35.0077) (width 0.2) (layer "F.Cu") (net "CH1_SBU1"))
 (segment (start 28.27 35.27) (end 28.9458 35.27) (width 0.2) (layer "F.Cu") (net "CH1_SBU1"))
 (segment (start 62.044 35.0077) (end 48.0594 35.0077) (width 0.2) (layer "F.Cu") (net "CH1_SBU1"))
 (segment (start 32.9731 33.9849) (end 33.5899 34.6017) (width 0.2) (layer "F.Cu") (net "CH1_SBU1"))
 (segment (start 30.2309 33.9849) (end 32.9731 33.9849) (width 0.2) (layer "F.Cu") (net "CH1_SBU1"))
 (segment (start 38.45 34) (end 38.45 34.6017) (width 0.2) (layer "F.Cu") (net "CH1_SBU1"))
 (segment (start 46.45 34) (end 47.0517 34) (width 0.2) (layer "F.Cu") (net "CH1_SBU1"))
 (segment (start 39.0517 34) (end 39.6534 33.3983) (width 0.2) (layer "F.Cu") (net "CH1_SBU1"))
 (segment (start 48.0594 35.0077) (end 47.0517 34) (width 0.2) (layer "F.Cu") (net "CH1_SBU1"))
 (segment (start 43.7966 41.3983) (end 36.9583 41.3983) (width 0.2) (layer "F.Cu") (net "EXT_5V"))
 (segment (start 36.9483 41.4083) (end 36.9483 42) (width 0.2) (layer "F.Cu") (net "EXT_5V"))
 (segment (start 61.55 50) (end 60.9483 50) (width 0.2) (layer "F.Cu") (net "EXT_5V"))
 (segment (start 60.3466 50.6017) (end 60.9483 50) (width 0.2) (layer "F.Cu") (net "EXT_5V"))
 (segment (start 45.1 42) (end 44.3983 42) (width 0.2) (layer "F.Cu") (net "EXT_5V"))
 (segment (start 45.55 50) (end 45.55 50.6017) (width 0.2) (layer "F.Cu") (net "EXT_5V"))
 (segment (start 37.55 42) (end 36.9483 42) (width 0.2) (layer "F.Cu") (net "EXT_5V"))
 (segment (start 36.9583 41.3983) (end 36.9483 41.4083) (width 0.2) (layer "F.Cu") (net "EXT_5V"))
 (segment (start 44.3983 42) (end 43.7966 41.3983) (width 0.2) (layer "F.Cu") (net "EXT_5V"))
 (segment (start 30.81 35.27) (end 36.9483 41.4083) (width 0.2) (layer "F.Cu") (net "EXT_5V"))
 (segment (start 45.55 50.6017) (end 60.3466 50.6017) (width 0.2) (layer "F.Cu") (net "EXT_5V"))
 (segment (start 38.0348 50) (end 45.55 50) (width 0.2) (layer "F.Cu") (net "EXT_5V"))
 (via (at 38.0348 50) (size 0.6) (drill 0.3) (layers "F.Cu" "B.Cu") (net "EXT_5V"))
 (segment (start 30.81 35.27) (end 38.0348 42.4948) (width 0.2) (layer "B.Cu") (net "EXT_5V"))
 (segment (start 38.0348 42.4948) (end 38.0348 50) (width 0.2) (layer "B.Cu") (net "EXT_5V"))
 (segment (start 29.54 34) (end 24.46 34) (width 0.2) (layer "B.Cu") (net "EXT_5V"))
 (segment (start 30.81 35.27) (end 29.54 34) (width 0.2) (layer "B.Cu") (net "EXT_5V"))
 (segment (start 24.46 34) (end 23.19 32.73) (width 0.2) (layer "B.Cu") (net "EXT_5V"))
 (segment (start 61.05 23.7982) (end 60.3444 23.7982) (width 0.2) (layer "F.Cu") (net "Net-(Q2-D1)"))
 (segment (start 61.55 34) (end 60.9483 34) (width 0.2) (layer "F.Cu") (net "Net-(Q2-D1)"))
 (segment (start 60.071 33.1227) (end 60.9483 34) (width 0.2) (layer "F.Cu") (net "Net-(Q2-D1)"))
 (segment (start 59.05 33.1227) (end 60.071 33.1227) (width 0.2) (layer "F.Cu") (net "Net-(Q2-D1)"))
 (segment (start 61.05 24.6999) (end 61.05 23.7982) (width 0.2) (layer "F.Cu") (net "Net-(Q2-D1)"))
 (via (at 59.05 33.1227) (size 0.6) (drill 0.3) (layers "F.Cu" "B.Cu") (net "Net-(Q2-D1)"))
 (via (at 60.3444 23.7982) (size 0.6) (drill 0.3) (layers "F.Cu" "B.Cu") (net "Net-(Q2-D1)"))
 (segment (start 59.05 33.1227) (end 59.05 25.0926) (width 0.2) (layer "B.Cu") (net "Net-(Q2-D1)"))
 (segment (start 59.05 25.0926) (end 60.3444 23.7982) (width 0.2) (layer "B.Cu") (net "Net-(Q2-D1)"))
 (segment (start 54.9017 27.05) (end 55.1206 27.05) (width 0.2) (layer "F.Cu") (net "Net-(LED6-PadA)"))
 (segment (start 46.45 50) (end 49.8886 50) (width 0.2) (layer "F.Cu") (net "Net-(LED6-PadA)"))
 (segment (start 54 27.05) (end 54.9017 27.05) (width 0.2) (layer "F.Cu") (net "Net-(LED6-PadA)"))
 (via (at 49.8886 50) (size 0.6) (drill 0.3) (layers "F.Cu" "B.Cu") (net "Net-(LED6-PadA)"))
 (via (at 55.1206 27.05) (size 0.6) (drill 0.3) (layers "F.Cu" "B.Cu") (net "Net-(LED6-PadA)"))
 (segment (start 49.8886 32.282) (end 49.8886 50) (width 0.2) (layer "B.Cu") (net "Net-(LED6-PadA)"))
 (segment (start 55.1206 27.05) (end 49.8886 32.282) (width 0.2) (layer "B.Cu") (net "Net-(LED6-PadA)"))
 (segment (start 35.8764 45.4164) (end 50.4681 45.4164) (width 0.2) (layer "F.Cu") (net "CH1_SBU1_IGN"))
 (segment (start 54.45 50) (end 54.45 49.3983) (width 0.2) (layer "F.Cu") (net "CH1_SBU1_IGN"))
 (segment (start 61.05 27.3001) (end 61.05 28.2018) (width 0.2) (layer "F.Cu") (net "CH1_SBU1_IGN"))
 (segment (start 61.05 28.2018) (end 56.5603 28.2018) (width 0.2) (layer "F.Cu") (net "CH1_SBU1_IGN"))
 (segment (start 47.1501 28.2018) (end 45.55 26.6017) (width 0.2) (layer "F.Cu") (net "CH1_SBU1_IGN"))
 (segment (start 50.4681 45.4164) (end 50.4999 45.3846) (width 0.2) (layer "F.Cu") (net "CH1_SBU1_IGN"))
 (segment (start 25.73 35.27) (end 35.8764 45.4164) (width 0.2) (layer "F.Cu") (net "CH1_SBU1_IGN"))
 (segment (start 45.55 26) (end 45.55 26.6017) (width 0.2) (layer "F.Cu") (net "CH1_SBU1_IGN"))
 (segment (start 50.4681 45.4164) (end 54.45 49.3983) (width 0.2) (layer "F.Cu") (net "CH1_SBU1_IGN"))
 (segment (start 56.5603 28.2018) (end 47.1501 28.2018) (width 0.2) (layer "F.Cu") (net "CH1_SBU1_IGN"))
 (via (at 56.5603 28.2018) (size 0.6) (drill 0.3) (layers "F.Cu" "B.Cu") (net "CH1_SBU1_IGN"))
 (via (at 50.4999 45.3846) (size 0.6) (drill 0.3) (layers "F.Cu" "B.Cu") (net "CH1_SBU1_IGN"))
 (segment (start 50.4999 34.2622) (end 56.5603 28.2018) (width 0.2) (layer "B.Cu") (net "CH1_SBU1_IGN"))
 (segment (start 50.4999 45.3846) (end 50.4999 34.2622) (width 0.2) (layer "B.Cu") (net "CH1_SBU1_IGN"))
 (segment (start 29.5278 31.4722) (end 34.4205 31.4722) (width 0.2) (layer "F.Cu") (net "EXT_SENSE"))
 (segment (start 34.4205 31.4722) (end 36.9483 34) (width 0.2) (layer "F.Cu") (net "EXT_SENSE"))
 (segment (start 28.27 32.73) (end 29.5278 31.4722) (width 0.2) (layer "F.Cu") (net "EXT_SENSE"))
 (segment (start 37.55 34) (end 36.9483 34) (width 0.2) (layer "F.Cu") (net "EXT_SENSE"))
 (segment (start 52.9483 50) (end 50.7635 47.8152) (width 0.2) (layer "F.Cu") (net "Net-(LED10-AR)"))
 (segment (start 50.7635 47.8152) (end 44.55 47.8152) (width 0.2) (layer "F.Cu") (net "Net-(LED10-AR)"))
 (segment (start 37.05 27) (end 37.7517 27) (width 0.2) (layer "F.Cu") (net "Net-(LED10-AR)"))
 (segment (start 53.55 50) (end 52.9483 50) (width 0.2) (layer "F.Cu") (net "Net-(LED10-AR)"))
 (segment (start 37.7517 27) (end 37.9567 27) (width 0.2) (layer "F.Cu") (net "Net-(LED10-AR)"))
 (via (at 37.9567 27) (size 0.6) (drill 0.3) (layers "F.Cu" "B.Cu") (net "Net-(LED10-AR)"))
 (via (at 44.55 47.8152) (size 0.6) (drill 0.3) (layers "F.Cu" "B.Cu") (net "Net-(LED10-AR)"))
 (segment (start 44.55 33.5933) (end 37.9567 27) (width 0.2) (layer "B.Cu") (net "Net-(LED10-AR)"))
 (segment (start 44.55 47.8152) (end 44.55 33.5933) (width 0.2) (layer "B.Cu") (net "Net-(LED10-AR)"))
 (segment (start 38.95 27) (end 39.6517 27) (width 0.2) (layer "F.Cu") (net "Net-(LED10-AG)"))
 (segment (start 39.6517 27) (end 41.4797 28.828) (width 0.2) (layer "F.Cu") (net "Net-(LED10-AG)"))
 (segment (start 53.55 34) (end 52.9483 34) (width 0.2) (layer "F.Cu") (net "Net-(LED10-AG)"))
 (segment (start 47.7763 28.828) (end 52.9483 34) (width 0.2) (layer "F.Cu") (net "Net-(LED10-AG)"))
 (segment (start 41.4797 28.828) (end 47.7763 28.828) (width 0.2) (layer "F.Cu") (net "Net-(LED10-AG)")))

